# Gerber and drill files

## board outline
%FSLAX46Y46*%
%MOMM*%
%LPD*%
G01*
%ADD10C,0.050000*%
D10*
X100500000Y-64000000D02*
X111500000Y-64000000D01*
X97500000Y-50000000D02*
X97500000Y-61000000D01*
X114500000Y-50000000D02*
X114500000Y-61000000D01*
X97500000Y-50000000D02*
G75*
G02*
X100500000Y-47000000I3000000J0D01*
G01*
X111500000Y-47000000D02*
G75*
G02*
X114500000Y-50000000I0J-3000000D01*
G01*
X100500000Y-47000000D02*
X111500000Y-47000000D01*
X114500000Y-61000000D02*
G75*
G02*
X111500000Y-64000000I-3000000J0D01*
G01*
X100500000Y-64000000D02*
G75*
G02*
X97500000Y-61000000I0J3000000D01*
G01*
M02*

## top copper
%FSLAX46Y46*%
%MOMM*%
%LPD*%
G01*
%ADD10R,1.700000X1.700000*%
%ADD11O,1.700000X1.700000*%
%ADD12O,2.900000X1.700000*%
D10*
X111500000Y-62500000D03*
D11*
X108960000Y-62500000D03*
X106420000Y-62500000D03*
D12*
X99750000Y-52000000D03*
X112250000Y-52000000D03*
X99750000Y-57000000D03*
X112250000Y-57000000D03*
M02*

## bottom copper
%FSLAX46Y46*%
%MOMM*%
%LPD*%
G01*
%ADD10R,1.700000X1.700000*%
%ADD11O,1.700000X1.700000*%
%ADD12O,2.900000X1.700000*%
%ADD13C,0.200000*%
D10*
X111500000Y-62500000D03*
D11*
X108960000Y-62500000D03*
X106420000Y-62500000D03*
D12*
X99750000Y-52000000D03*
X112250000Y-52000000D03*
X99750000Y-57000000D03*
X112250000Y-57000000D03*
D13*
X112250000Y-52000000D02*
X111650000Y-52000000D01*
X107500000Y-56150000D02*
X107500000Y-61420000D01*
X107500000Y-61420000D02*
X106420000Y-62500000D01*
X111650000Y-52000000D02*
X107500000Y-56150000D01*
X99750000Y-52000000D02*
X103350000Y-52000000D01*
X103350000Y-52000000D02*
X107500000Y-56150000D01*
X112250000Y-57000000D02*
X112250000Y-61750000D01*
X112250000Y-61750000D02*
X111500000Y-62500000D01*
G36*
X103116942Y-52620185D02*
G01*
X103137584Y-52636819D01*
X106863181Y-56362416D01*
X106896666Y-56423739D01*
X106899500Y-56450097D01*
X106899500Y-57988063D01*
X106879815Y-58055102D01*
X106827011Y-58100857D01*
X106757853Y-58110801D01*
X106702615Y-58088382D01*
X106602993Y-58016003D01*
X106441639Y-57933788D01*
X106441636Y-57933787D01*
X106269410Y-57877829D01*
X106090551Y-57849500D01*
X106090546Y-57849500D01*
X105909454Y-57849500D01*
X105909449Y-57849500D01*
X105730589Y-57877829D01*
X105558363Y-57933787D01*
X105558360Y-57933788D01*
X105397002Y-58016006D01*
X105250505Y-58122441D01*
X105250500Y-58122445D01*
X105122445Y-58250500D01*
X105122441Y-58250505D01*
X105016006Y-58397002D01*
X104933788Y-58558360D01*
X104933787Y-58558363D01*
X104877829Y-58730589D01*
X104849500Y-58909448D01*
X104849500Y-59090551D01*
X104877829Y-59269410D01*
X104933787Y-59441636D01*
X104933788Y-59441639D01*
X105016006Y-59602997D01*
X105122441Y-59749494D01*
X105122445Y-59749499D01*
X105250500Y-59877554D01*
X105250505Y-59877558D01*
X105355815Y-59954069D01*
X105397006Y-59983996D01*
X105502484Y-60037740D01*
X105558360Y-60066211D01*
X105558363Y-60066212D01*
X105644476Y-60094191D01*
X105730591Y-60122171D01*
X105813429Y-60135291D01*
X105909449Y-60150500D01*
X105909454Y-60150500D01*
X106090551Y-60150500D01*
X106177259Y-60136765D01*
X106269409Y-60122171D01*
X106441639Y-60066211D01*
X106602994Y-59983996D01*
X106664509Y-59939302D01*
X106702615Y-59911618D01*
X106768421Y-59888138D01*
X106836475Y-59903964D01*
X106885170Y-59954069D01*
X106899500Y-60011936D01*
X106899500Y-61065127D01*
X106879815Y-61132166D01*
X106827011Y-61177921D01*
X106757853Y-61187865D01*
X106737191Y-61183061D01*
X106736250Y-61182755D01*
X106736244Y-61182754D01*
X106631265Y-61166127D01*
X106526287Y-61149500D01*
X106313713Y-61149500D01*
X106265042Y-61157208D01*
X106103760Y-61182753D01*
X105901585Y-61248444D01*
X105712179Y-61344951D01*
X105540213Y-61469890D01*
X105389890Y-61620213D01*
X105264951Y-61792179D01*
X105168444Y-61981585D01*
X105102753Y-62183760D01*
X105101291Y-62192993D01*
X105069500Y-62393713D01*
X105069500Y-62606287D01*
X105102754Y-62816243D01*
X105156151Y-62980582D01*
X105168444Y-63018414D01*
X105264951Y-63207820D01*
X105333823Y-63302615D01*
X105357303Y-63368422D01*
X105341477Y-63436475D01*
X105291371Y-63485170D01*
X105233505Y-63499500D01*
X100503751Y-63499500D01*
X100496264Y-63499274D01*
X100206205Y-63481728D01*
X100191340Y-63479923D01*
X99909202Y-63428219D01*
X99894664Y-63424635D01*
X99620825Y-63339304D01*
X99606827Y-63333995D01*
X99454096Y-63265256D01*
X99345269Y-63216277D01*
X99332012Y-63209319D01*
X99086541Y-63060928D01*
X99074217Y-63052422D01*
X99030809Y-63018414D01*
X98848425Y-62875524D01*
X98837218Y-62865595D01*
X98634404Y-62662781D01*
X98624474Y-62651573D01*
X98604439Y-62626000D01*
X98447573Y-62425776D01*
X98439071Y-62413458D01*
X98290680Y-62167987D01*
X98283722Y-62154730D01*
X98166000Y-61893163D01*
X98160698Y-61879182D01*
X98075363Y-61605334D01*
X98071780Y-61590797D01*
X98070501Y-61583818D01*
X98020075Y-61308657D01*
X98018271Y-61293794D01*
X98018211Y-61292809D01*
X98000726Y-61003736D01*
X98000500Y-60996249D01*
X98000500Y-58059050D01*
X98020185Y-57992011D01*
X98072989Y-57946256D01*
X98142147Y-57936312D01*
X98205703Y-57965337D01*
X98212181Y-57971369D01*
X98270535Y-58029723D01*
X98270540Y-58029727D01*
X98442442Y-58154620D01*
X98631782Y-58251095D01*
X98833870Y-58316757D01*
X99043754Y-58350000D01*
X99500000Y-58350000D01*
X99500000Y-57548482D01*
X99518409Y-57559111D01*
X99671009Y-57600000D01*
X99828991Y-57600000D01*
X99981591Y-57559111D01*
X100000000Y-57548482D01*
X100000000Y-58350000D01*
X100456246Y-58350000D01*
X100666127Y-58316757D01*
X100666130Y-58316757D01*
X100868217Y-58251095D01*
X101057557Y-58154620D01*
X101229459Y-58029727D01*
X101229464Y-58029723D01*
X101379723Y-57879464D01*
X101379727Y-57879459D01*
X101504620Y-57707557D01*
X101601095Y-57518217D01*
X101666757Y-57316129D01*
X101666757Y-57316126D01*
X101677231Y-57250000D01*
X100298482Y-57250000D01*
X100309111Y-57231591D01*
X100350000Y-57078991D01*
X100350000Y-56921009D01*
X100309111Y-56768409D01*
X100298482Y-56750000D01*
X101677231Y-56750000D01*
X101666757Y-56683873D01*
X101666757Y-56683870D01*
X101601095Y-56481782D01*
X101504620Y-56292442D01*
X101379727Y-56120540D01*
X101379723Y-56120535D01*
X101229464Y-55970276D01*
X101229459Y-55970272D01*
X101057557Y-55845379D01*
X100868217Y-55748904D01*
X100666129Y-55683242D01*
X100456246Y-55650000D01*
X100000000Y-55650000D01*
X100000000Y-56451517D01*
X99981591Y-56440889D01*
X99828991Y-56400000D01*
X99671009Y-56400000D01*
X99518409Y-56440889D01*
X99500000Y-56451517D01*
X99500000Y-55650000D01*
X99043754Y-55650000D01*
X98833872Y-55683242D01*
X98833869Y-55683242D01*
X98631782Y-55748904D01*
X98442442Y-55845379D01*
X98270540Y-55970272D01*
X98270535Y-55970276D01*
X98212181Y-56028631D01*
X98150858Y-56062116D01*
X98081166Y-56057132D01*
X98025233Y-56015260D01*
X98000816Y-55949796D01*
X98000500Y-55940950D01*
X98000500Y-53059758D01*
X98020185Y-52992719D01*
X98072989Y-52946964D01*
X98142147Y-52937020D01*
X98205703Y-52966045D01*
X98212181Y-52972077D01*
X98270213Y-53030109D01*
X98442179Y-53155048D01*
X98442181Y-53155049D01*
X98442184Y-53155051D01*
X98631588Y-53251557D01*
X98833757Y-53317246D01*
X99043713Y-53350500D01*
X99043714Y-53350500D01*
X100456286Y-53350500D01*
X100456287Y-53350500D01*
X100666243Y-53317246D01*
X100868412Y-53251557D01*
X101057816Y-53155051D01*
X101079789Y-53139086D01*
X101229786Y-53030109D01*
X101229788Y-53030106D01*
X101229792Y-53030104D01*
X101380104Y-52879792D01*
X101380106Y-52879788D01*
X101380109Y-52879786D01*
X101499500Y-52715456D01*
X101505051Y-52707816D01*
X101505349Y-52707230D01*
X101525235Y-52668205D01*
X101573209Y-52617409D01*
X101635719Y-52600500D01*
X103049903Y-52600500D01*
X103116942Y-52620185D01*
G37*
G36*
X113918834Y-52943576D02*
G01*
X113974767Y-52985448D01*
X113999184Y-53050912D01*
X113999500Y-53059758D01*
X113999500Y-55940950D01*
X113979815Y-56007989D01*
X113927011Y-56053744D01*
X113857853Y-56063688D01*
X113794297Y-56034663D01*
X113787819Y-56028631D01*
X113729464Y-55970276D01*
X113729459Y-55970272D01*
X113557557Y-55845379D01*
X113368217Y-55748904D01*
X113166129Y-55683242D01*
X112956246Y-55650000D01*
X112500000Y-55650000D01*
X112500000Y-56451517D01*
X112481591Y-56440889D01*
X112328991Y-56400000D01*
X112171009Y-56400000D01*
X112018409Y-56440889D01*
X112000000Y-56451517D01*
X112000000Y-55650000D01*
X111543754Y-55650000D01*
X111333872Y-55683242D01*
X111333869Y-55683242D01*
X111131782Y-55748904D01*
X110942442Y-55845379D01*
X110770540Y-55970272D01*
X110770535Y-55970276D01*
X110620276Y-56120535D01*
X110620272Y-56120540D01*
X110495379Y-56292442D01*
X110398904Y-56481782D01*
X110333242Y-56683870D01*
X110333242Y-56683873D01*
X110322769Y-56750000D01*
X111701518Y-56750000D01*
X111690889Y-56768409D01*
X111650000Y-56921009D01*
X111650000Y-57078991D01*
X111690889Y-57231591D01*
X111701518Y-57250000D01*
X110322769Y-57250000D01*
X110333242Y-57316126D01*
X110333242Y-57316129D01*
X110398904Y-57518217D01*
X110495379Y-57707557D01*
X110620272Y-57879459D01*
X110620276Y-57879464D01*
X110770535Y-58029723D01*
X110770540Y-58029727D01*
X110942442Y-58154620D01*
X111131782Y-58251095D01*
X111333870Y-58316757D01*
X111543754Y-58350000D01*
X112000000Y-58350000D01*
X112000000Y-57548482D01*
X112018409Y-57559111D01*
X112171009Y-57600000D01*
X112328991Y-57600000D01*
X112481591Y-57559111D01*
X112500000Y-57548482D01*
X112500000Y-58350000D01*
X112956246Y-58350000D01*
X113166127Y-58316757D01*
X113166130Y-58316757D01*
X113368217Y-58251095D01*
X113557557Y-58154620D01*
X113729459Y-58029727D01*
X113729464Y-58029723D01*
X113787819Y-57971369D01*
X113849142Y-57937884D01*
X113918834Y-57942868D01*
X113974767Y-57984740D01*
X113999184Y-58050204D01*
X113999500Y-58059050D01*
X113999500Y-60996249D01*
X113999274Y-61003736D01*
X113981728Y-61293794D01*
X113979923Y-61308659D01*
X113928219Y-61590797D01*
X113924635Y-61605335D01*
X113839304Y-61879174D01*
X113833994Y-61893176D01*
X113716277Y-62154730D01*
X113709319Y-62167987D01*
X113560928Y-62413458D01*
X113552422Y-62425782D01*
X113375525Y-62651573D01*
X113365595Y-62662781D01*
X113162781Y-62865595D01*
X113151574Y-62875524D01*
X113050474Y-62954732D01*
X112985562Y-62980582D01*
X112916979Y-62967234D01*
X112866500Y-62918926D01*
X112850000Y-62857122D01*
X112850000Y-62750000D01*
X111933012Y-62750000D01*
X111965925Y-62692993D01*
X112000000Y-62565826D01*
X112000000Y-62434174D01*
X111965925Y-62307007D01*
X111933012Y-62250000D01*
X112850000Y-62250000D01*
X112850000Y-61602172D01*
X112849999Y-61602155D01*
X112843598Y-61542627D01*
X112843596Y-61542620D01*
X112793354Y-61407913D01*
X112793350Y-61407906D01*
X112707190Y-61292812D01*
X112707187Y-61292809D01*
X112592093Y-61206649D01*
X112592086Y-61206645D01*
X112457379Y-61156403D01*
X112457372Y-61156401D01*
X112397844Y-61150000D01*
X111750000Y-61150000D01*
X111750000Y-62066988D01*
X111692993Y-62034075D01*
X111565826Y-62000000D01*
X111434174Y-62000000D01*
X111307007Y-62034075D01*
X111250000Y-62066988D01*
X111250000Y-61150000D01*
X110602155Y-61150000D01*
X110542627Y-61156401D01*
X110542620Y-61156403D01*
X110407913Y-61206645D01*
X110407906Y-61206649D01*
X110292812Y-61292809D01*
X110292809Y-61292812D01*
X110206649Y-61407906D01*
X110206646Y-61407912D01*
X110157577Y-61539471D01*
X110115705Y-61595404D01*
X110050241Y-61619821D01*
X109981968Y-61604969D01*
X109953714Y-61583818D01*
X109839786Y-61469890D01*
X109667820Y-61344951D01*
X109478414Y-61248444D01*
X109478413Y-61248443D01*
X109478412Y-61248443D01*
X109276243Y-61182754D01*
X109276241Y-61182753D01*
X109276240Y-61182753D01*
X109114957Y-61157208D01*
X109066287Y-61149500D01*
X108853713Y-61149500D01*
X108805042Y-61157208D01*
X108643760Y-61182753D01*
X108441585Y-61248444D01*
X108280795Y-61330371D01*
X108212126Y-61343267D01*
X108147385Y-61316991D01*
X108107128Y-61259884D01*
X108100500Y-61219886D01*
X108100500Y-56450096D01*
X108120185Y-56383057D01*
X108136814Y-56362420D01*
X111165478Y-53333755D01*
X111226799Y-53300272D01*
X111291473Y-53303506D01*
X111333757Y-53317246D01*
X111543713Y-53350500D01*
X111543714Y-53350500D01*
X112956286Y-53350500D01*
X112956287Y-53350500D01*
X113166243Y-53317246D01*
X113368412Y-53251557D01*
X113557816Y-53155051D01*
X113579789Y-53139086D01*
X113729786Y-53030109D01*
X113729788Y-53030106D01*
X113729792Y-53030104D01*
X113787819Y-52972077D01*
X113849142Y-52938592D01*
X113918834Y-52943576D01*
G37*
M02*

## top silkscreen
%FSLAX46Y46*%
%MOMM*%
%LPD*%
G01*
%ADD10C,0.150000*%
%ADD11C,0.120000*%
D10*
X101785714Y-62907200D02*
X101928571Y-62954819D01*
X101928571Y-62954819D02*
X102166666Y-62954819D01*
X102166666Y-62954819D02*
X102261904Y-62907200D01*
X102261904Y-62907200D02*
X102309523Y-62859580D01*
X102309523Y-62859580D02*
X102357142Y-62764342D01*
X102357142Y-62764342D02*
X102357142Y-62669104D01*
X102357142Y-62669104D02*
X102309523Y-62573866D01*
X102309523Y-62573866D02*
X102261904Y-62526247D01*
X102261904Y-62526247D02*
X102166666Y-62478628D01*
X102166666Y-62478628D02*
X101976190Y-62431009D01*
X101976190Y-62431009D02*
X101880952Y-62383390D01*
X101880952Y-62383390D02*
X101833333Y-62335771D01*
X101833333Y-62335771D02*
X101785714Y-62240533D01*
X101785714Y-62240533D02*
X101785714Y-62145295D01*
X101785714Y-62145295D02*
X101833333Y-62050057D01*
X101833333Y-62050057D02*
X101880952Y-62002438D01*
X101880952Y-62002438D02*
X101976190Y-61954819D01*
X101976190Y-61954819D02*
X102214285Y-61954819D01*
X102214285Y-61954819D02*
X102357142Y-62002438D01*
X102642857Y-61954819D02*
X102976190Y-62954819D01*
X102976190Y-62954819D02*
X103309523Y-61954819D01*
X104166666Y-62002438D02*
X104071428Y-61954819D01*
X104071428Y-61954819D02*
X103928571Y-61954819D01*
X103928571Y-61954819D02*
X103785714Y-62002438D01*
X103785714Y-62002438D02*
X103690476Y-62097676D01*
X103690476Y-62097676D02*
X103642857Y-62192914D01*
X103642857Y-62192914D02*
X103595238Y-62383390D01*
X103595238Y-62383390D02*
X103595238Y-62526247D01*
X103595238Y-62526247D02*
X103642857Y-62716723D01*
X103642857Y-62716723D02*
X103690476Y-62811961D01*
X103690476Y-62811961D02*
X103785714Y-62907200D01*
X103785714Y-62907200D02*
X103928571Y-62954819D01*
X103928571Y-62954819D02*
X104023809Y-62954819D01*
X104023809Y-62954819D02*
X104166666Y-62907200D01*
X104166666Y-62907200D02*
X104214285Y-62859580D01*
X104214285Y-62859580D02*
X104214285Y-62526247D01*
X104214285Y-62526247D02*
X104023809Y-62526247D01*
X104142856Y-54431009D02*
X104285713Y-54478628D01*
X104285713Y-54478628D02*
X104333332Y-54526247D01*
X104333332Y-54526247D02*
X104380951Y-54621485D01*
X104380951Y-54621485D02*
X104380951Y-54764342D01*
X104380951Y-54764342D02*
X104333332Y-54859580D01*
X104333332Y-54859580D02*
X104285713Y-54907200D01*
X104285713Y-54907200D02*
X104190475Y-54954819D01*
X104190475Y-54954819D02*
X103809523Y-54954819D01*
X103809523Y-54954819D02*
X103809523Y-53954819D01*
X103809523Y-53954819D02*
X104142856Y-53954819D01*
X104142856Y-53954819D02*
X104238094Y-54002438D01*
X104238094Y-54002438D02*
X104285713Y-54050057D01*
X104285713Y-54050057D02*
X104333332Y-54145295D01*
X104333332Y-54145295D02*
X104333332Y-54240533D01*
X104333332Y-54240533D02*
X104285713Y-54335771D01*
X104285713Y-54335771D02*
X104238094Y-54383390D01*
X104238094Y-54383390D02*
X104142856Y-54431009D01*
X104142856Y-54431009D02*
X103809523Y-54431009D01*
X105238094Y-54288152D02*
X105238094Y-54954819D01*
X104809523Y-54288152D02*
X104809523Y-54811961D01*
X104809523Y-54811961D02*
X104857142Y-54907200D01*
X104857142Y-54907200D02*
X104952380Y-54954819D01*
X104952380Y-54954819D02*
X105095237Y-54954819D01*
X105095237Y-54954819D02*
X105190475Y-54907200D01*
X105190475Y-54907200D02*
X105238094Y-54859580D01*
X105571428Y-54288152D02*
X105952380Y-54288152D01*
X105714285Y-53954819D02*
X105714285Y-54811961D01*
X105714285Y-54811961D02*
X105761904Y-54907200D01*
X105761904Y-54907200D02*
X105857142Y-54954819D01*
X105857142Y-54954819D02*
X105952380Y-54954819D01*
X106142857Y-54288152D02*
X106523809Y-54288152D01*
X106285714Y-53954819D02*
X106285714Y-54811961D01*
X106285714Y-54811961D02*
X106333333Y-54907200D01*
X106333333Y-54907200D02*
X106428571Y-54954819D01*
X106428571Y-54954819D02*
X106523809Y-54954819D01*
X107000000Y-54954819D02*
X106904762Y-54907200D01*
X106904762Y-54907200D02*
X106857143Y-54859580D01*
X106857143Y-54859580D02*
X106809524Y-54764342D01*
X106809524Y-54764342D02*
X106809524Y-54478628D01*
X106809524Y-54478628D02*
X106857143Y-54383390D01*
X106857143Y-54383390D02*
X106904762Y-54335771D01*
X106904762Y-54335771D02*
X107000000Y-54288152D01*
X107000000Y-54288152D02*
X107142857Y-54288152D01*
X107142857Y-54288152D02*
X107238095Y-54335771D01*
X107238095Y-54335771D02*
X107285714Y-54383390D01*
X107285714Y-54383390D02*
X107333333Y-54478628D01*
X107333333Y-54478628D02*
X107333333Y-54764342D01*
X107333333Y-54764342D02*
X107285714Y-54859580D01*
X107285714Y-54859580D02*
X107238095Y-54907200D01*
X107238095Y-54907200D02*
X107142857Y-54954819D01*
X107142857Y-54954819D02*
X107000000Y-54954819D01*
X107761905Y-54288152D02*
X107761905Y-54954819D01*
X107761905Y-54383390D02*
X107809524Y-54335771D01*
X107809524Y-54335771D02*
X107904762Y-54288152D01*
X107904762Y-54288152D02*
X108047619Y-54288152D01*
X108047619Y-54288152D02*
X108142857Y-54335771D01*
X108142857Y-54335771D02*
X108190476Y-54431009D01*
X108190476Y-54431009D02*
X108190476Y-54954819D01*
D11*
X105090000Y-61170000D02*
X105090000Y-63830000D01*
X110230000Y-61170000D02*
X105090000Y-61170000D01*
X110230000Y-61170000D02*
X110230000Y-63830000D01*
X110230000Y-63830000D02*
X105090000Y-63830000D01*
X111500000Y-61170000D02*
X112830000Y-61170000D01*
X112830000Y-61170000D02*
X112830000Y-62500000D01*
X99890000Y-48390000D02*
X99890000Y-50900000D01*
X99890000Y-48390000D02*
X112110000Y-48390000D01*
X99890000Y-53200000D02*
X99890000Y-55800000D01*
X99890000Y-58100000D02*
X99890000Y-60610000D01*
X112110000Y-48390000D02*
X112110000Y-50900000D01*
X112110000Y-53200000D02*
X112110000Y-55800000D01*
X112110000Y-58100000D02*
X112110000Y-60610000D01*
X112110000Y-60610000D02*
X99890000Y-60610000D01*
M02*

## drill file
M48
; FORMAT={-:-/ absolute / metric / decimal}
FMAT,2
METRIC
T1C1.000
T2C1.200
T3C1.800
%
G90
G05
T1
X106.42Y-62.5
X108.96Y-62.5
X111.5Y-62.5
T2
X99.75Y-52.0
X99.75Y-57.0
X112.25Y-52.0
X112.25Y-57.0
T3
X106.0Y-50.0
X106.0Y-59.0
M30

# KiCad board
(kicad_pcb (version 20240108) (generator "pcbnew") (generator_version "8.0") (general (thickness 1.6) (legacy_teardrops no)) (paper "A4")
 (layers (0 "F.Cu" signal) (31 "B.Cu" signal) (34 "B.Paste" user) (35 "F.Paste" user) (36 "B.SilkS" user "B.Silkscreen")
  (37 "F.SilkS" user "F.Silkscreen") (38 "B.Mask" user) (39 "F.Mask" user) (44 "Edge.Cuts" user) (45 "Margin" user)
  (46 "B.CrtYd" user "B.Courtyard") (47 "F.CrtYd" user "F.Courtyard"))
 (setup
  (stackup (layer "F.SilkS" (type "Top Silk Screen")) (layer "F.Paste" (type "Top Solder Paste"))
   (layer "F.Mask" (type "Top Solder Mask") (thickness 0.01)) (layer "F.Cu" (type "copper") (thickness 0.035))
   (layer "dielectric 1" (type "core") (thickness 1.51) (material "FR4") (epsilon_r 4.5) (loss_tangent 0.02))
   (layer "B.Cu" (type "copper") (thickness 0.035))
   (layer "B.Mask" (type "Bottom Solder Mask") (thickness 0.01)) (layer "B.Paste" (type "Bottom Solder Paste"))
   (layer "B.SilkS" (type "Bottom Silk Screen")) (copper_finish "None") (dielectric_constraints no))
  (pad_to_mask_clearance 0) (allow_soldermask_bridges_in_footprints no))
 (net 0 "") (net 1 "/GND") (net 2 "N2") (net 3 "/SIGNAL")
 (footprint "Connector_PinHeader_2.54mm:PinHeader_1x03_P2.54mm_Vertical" (layer "F.Cu") (at 111.5 62.5 -90)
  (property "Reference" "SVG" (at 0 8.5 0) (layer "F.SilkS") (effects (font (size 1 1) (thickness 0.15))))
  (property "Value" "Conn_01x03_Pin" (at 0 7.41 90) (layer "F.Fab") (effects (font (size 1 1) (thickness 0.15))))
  (fp_line (start -1.33 6.41) (end 1.33 6.41) (stroke (width 0.12) (type solid)) (layer "F.SilkS"))
  (fp_line (start -1.33 1.27) (end -1.33 6.41) (stroke (width 0.12) (type solid)) (layer "F.SilkS"))
  (fp_line (start -1.33 1.27) (end 1.33 1.27) (stroke (width 0.12) (type solid)) (layer "F.SilkS"))
  (fp_line (start 1.33 1.27) (end 1.33 6.41) (stroke (width 0.12) (type solid)) (layer "F.SilkS"))
  (fp_line (start -1.33 0) (end -1.33 -1.33) (stroke (width 0.12) (type solid)) (layer "F.SilkS"))
  (fp_line (start -1.33 -1.33) (end 0 -1.33) (stroke (width 0.12) (type solid)) (layer "F.SilkS"))
  (pad "1" thru_hole rect (at 0 0 270) (size 1.7 1.7) (drill 1) (layers "*.Cu" "*.Mask") (remove_unused_layers no) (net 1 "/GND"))
  (pad "2" thru_hole oval (at 0 2.54 270) (size 1.7 1.7) (drill 1) (layers "*.Cu" "*.Mask") (remove_unused_layers no) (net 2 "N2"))
  (pad "3" thru_hole oval (at 0 5.08 270) (size 1.7 1.7) (drill 1) (layers "*.Cu" "*.Mask") (remove_unused_layers no) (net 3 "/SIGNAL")))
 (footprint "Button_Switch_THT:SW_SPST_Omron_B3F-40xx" (layer "F.Cu") (at 99.75 52)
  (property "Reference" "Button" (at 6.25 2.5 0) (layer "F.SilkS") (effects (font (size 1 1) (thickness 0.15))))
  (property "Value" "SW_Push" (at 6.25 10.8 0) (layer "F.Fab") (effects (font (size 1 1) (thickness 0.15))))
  (fp_line (start 0.14 -3.61) (end 0.14 -1.1) (stroke (width 0.12) (type default)) (layer "F.SilkS"))
  (fp_line (start 0.14 -3.61) (end 12.36 -3.61) (stroke (width 0.12) (type default)) (layer "F.SilkS"))
  (fp_line (start 0.14 1.2) (end 0.14 3.8) (stroke (width 0.12) (type default)) (layer "F.SilkS"))
  (fp_line (start 0.14 6.1) (end 0.14 8.61) (stroke (width 0.12) (type default)) (layer "F.SilkS"))
  (fp_line (start 12.36 -3.61) (end 12.36 -1.1) (stroke (width 0.12) (type default)) (layer "F.SilkS"))
  (fp_line (start 12.36 1.2) (end 12.36 3.8) (stroke (width 0.12) (type default)) (layer "F.SilkS"))
  (fp_line (start 12.36 6.1) (end 12.36 8.61) (stroke (width 0.12) (type default)) (layer "F.SilkS"))
  (fp_line (start 12.36 8.61) (end 0.14 8.61) (stroke (width 0.12) (type default)) (layer "F.SilkS"))
  (pad "" np_thru_hole circle (at 6.25 -2) (size 1.8 1.8) (drill 1.8) (layers "F&B.Cu" "*.Mask"))
  (pad "" np_thru_hole circle (at 6.25 7) (size 1.8 1.8) (drill 1.8) (layers "F&B.Cu" "*.Mask"))
  (pad "1" thru_hole oval (at 0 0) (size 2.9 1.7) (drill 1.2) (layers "*.Cu" "*.Mask") (remove_unused_layers no) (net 3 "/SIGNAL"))
  (pad "1" thru_hole oval (at 12.5 0) (size 2.9 1.7) (drill 1.2) (layers "*.Cu" "*.Mask") (remove_unused_layers no) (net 3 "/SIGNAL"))
  (pad "2" thru_hole oval (at 0 5) (size 2.9 1.7) (drill 1.2) (layers "*.Cu" "*.Mask") (remove_unused_layers no) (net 1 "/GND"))
  (pad "2" thru_hole oval (at 12.5 5) (size 2.9 1.7) (drill 1.2) (layers "*.Cu" "*.Mask") (remove_unused_layers no) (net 1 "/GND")))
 (gr_line (start 100.5 64) (end 111.5 64) (locked yes) (stroke (width 0.05) (type default)) (layer "Edge.Cuts"))
 (gr_line (start 97.5 50) (end 97.5 61) (locked yes) (stroke (width 0.05) (type default)) (layer "Edge.Cuts"))
 (gr_line (start 114.5 50) (end 114.5 61) (locked yes) (stroke (width 0.05) (type default)) (layer "Edge.Cuts"))
 (gr_arc (start 97.5 50) (mid 98.37868 47.87868) (end 100.5 47) (locked yes) (stroke (width 0.05) (type default)) (layer "Edge.Cuts"))
 (gr_arc (start 111.5 47) (mid 113.62132 47.87868) (end 114.5 50) (locked yes) (stroke (width 0.05) (type default)) (layer "Edge.Cuts"))
 (gr_line (start 100.5 47) (end 111.5 47) (locked yes) (stroke (width 0.05) (type default)) (layer "Edge.Cuts"))
 (gr_arc (start 114.5 61) (mid 113.62132 63.12132) (end 111.5 64) (locked yes) (stroke (width 0.05) (type default)) (layer "Edge.Cuts"))
 (gr_arc (start 100.5 64) (mid 98.37868 63.12132) (end 97.5 61) (locked yes) (stroke (width 0.05) (type default)) (layer "Edge.Cuts"))
 (segment (start 112.25 52) (end 111.65 52) (width 0.2) (layer "B.Cu") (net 3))
 (segment (start 107.5 56.15) (end 107.5 61.42) (width 0.2) (layer "B.Cu") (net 3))
 (segment (start 107.5 61.42) (end 106.42 62.5) (width 0.2) (layer "B.Cu") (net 3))
 (segment (start 111.65 52) (end 107.5 56.15) (width 0.2) (layer "B.Cu") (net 3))
 (segment (start 99.75 52) (end 103.35 52) (width 0.2) (layer "B.Cu") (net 3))
 (segment (start 103.35 52) (end 107.5 56.15) (width 0.2) (layer "B.Cu") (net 3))
 (segment (start 112.25 57) (end 112.25 61.75) (width 0.2) (layer "B.Cu") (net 1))
 (segment (start 112.25 61.75) (end 111.5 62.5) (width 0.2) (layer "B.Cu") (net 1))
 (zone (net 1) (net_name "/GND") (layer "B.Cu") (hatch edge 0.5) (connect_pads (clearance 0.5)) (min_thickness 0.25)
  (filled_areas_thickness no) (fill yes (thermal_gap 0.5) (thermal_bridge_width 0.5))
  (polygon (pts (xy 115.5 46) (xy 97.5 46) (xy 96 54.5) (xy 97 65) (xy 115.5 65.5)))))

